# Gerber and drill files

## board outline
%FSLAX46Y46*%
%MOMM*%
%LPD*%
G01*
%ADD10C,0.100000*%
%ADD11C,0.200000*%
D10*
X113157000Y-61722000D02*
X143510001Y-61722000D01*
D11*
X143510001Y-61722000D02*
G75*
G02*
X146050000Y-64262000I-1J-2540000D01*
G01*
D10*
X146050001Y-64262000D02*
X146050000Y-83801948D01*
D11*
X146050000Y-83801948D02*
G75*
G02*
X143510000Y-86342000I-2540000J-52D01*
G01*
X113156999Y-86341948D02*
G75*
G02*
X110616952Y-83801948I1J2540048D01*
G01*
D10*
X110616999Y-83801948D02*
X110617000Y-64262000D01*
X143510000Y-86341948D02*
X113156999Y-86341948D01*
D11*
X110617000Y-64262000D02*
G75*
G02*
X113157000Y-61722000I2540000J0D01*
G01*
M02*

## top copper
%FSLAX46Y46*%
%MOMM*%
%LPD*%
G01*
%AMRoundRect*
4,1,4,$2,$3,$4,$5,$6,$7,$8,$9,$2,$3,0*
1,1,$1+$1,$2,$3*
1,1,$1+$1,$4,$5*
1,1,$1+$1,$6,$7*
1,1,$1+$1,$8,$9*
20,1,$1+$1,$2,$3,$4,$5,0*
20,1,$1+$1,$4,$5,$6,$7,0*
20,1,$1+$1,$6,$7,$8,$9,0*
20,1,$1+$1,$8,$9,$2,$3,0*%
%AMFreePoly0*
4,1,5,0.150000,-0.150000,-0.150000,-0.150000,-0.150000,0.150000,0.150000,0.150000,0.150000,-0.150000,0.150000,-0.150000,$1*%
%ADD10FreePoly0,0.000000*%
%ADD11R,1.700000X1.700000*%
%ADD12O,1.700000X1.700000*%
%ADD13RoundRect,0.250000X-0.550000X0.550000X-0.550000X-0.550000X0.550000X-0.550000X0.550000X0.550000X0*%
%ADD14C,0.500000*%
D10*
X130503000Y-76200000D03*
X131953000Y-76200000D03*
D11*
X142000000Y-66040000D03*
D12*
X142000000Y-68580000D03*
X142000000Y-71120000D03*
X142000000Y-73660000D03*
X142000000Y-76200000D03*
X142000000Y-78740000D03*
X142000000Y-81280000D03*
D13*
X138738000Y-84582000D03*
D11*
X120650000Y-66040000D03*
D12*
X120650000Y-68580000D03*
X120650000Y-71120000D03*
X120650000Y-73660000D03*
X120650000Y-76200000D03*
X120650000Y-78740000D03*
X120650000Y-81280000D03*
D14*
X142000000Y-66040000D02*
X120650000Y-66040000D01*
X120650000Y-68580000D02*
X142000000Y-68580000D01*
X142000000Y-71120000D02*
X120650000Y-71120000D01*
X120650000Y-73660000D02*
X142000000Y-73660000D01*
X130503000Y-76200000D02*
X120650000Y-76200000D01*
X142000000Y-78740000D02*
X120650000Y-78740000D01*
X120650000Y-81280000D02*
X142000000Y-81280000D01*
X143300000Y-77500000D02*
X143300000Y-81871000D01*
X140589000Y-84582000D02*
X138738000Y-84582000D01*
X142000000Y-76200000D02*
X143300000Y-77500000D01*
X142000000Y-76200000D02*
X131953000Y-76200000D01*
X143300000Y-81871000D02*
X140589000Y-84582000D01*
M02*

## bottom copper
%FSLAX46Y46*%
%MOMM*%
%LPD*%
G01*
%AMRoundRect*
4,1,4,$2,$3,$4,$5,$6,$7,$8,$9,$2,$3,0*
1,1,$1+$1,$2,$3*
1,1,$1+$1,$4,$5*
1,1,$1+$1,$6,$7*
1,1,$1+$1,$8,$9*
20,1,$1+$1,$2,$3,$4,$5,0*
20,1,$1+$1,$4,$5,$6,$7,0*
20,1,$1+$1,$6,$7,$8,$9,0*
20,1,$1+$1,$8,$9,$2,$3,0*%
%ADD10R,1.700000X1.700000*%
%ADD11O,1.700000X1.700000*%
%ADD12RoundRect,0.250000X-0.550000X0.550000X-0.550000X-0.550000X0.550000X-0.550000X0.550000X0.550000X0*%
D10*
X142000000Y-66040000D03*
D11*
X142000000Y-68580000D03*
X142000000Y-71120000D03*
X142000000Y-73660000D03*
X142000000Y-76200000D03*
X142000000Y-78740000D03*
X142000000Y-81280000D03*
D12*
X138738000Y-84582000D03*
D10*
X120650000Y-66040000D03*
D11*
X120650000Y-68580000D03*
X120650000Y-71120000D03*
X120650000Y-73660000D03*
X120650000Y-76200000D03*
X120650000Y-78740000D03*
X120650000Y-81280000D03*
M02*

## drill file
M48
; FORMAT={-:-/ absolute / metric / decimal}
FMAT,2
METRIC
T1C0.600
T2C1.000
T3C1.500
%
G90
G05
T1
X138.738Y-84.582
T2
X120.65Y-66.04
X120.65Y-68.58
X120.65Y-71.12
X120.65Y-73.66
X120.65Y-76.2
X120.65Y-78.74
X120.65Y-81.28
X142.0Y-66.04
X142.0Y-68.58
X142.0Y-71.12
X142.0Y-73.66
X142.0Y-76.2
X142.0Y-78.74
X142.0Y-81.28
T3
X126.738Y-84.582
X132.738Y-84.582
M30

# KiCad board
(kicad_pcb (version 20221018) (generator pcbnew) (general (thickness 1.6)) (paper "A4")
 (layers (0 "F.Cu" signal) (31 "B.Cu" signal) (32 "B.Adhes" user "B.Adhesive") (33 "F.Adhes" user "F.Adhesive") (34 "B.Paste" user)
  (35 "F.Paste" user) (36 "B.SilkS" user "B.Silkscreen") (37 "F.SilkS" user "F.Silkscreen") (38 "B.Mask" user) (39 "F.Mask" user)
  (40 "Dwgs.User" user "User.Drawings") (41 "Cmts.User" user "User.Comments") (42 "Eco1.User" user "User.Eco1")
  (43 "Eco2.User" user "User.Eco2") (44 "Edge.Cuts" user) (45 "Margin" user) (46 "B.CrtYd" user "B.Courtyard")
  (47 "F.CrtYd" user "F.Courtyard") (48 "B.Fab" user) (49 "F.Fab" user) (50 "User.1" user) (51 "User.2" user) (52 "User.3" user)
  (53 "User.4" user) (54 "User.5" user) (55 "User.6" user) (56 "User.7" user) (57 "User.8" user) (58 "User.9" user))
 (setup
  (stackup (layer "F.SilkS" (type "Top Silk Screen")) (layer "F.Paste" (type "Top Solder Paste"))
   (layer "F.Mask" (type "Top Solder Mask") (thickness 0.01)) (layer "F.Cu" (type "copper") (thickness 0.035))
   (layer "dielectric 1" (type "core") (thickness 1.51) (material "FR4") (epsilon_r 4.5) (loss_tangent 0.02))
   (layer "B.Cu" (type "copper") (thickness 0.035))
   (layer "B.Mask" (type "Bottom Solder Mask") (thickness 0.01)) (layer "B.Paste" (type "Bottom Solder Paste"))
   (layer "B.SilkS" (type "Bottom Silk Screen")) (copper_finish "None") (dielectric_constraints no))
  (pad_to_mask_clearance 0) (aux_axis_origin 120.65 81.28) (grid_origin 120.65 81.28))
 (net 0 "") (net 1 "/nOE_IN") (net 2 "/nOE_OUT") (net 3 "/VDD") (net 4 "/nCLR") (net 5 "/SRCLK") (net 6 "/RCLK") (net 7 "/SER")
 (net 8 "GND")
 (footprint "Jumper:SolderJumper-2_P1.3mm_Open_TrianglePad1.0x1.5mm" (layer "F.Cu") (at 131.228 76.2)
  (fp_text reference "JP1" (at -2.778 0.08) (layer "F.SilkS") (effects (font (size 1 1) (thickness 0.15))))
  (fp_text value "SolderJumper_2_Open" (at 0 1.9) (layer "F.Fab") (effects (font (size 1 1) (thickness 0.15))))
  (pad "1" smd custom (at -0.725 0) (size 0.3 0.3) (layers "F.Cu" "F.Mask") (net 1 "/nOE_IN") (zone_connect 2) (thermal_bridge_angle 45)
   (options (clearance outline) (anchor rect)) (primitives))
  (pad "2" smd custom (at 0.725 0) (size 0.3 0.3) (layers "F.Cu" "F.Mask") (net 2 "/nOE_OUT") (zone_connect 2) (thermal_bridge_angle 45)
   (options (clearance outline) (anchor rect)) (primitives)))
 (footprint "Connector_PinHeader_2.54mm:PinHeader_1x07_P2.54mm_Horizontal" (layer "F.Cu") (at 142 66.04)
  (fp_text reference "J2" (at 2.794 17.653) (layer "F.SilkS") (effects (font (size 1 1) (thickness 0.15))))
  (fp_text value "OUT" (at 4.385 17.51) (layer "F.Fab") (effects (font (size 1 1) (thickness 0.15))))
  (pad "1" thru_hole rect (at 0 0) (size 1.7 1.7) (drill 1) (layers "*.Cu" "*.Mask") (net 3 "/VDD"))
  (pad "2" thru_hole oval (at 0 2.54) (size 1.7 1.7) (drill 1) (layers "*.Cu" "*.Mask") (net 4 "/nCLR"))
  (pad "3" thru_hole oval (at 0 5.08) (size 1.7 1.7) (drill 1) (layers "*.Cu" "*.Mask") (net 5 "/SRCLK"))
  (pad "4" thru_hole oval (at 0 7.62) (size 1.7 1.7) (drill 1) (layers "*.Cu" "*.Mask") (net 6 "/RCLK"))
  (pad "5" thru_hole oval (at 0 10.16) (size 1.7 1.7) (drill 1) (layers "*.Cu" "*.Mask") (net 2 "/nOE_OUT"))
  (pad "6" thru_hole oval (at 0 12.7) (size 1.7 1.7) (drill 1) (layers "*.Cu" "*.Mask") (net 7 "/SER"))
  (pad "7" thru_hole oval (at 0 15.24) (size 1.7 1.7) (drill 1) (layers "*.Cu" "*.Mask") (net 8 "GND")))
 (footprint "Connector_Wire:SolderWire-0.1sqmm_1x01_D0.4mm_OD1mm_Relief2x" (layer "F.Cu") (at 138.738 84.582 -90)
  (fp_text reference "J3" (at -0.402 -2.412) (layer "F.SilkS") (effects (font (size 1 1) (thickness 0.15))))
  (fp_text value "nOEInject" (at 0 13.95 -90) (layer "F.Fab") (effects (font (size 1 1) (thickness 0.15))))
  (pad "" np_thru_hole circle (at 0 6 270) (size 1.5 1.5) (drill 1.5) (layers "*.Cu" "*.Mask"))
  (pad "" np_thru_hole circle (at 0 12 270) (size 1.5 1.5) (drill 1.5) (layers "*.Cu" "*.Mask"))
  (pad "1" thru_hole roundrect (at 0 0 270) (size 1.6 1.6) (drill 0.6) (layers "*.Cu" "*.Mask") (roundrect_rratio 0.15625)
   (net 2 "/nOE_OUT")))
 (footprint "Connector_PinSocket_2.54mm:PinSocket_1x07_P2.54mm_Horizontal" (layer "F.Cu") (at 120.65 66.04)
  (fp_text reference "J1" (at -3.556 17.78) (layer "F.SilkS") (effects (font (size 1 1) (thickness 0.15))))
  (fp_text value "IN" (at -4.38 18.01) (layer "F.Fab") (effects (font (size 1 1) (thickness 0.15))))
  (pad "1" thru_hole rect (at 0 0) (size 1.7 1.7) (drill 1) (layers "*.Cu" "*.Mask") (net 3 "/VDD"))
  (pad "2" thru_hole oval (at 0 2.54) (size 1.7 1.7) (drill 1) (layers "*.Cu" "*.Mask") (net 4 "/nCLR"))
  (pad "3" thru_hole oval (at 0 5.08) (size 1.7 1.7) (drill 1) (layers "*.Cu" "*.Mask") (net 5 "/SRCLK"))
  (pad "4" thru_hole oval (at 0 7.62) (size 1.7 1.7) (drill 1) (layers "*.Cu" "*.Mask") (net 6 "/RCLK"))
  (pad "5" thru_hole oval (at 0 10.16) (size 1.7 1.7) (drill 1) (layers "*.Cu" "*.Mask") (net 1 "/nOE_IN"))
  (pad "6" thru_hole oval (at 0 12.7) (size 1.7 1.7) (drill 1) (layers "*.Cu" "*.Mask") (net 7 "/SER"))
  (pad "7" thru_hole oval (at 0 15.24) (size 1.7 1.7) (drill 1) (layers "*.Cu" "*.Mask") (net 8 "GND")))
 (gr_line (start 113.157 61.722) (end 143.510001 61.722) (stroke (width 0.1) (type default)) (layer "Edge.Cuts"))
 (gr_arc (start 143.510001 61.722) (mid 145.306052 62.465949) (end 146.050001 64.262) (stroke (width 0.2) (type default))
  (layer "Edge.Cuts"))
 (gr_line (start 146.050001 64.262) (end 146.05 83.801948) (stroke (width 0.1) (type default)) (layer "Edge.Cuts"))
 (gr_arc (start 146.05 83.801948) (mid 145.306052 85.598) (end 143.51 86.341948) (stroke (width 0.2) (type default)) (layer "Edge.Cuts"))
 (gr_arc (start 113.156999 86.341948) (mid 111.360948 85.597999) (end 110.616999 83.801948) (stroke (width 0.2) (type default))
  (layer "Edge.Cuts"))
 (gr_line (start 110.616999 83.801948) (end 110.617 64.262) (stroke (width 0.1) (type default)) (layer "Edge.Cuts"))
 (gr_line (start 143.51 86.341948) (end 113.156999 86.341948) (stroke (width 0.1) (type default)) (layer "Edge.Cuts"))
 (gr_arc (start 110.617 64.262) (mid 111.360948 62.465948) (end 113.157 61.722) (stroke (width 0.2) (type default)) (layer "Edge.Cuts"))
 (segment (start 142 66.04) (end 120.65 66.04) (width 0.5) (layer "F.Cu") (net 3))
 (segment (start 120.65 68.58) (end 142 68.58) (width 0.5) (layer "F.Cu") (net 4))
 (segment (start 142 71.12) (end 120.65 71.12) (width 0.5) (layer "F.Cu") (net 5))
 (segment (start 120.65 73.66) (end 142 73.66) (width 0.5) (layer "F.Cu") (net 6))
 (segment (start 130.503 76.2) (end 120.65 76.2) (width 0.5) (layer "F.Cu") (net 1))
 (segment (start 142 78.74) (end 120.65 78.74) (width 0.5) (layer "F.Cu") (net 7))
 (segment (start 120.65 81.28) (end 142 81.28) (width 0.5) (layer "F.Cu") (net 8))
 (segment (start 143.3 77.5) (end 143.3 81.871) (width 0.5) (layer "F.Cu") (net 2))
 (segment (start 140.589 84.582) (end 138.738 84.582) (width 0.5) (layer "F.Cu") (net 2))
 (segment (start 142 76.2) (end 143.3 77.5) (width 0.5) (layer "F.Cu") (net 2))
 (segment (start 142 76.2) (end 131.953 76.2) (width 0.5) (layer "F.Cu") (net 2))
 (segment (start 143.3 81.871) (end 140.589 84.582) (width 0.5) (layer "F.Cu") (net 2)))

